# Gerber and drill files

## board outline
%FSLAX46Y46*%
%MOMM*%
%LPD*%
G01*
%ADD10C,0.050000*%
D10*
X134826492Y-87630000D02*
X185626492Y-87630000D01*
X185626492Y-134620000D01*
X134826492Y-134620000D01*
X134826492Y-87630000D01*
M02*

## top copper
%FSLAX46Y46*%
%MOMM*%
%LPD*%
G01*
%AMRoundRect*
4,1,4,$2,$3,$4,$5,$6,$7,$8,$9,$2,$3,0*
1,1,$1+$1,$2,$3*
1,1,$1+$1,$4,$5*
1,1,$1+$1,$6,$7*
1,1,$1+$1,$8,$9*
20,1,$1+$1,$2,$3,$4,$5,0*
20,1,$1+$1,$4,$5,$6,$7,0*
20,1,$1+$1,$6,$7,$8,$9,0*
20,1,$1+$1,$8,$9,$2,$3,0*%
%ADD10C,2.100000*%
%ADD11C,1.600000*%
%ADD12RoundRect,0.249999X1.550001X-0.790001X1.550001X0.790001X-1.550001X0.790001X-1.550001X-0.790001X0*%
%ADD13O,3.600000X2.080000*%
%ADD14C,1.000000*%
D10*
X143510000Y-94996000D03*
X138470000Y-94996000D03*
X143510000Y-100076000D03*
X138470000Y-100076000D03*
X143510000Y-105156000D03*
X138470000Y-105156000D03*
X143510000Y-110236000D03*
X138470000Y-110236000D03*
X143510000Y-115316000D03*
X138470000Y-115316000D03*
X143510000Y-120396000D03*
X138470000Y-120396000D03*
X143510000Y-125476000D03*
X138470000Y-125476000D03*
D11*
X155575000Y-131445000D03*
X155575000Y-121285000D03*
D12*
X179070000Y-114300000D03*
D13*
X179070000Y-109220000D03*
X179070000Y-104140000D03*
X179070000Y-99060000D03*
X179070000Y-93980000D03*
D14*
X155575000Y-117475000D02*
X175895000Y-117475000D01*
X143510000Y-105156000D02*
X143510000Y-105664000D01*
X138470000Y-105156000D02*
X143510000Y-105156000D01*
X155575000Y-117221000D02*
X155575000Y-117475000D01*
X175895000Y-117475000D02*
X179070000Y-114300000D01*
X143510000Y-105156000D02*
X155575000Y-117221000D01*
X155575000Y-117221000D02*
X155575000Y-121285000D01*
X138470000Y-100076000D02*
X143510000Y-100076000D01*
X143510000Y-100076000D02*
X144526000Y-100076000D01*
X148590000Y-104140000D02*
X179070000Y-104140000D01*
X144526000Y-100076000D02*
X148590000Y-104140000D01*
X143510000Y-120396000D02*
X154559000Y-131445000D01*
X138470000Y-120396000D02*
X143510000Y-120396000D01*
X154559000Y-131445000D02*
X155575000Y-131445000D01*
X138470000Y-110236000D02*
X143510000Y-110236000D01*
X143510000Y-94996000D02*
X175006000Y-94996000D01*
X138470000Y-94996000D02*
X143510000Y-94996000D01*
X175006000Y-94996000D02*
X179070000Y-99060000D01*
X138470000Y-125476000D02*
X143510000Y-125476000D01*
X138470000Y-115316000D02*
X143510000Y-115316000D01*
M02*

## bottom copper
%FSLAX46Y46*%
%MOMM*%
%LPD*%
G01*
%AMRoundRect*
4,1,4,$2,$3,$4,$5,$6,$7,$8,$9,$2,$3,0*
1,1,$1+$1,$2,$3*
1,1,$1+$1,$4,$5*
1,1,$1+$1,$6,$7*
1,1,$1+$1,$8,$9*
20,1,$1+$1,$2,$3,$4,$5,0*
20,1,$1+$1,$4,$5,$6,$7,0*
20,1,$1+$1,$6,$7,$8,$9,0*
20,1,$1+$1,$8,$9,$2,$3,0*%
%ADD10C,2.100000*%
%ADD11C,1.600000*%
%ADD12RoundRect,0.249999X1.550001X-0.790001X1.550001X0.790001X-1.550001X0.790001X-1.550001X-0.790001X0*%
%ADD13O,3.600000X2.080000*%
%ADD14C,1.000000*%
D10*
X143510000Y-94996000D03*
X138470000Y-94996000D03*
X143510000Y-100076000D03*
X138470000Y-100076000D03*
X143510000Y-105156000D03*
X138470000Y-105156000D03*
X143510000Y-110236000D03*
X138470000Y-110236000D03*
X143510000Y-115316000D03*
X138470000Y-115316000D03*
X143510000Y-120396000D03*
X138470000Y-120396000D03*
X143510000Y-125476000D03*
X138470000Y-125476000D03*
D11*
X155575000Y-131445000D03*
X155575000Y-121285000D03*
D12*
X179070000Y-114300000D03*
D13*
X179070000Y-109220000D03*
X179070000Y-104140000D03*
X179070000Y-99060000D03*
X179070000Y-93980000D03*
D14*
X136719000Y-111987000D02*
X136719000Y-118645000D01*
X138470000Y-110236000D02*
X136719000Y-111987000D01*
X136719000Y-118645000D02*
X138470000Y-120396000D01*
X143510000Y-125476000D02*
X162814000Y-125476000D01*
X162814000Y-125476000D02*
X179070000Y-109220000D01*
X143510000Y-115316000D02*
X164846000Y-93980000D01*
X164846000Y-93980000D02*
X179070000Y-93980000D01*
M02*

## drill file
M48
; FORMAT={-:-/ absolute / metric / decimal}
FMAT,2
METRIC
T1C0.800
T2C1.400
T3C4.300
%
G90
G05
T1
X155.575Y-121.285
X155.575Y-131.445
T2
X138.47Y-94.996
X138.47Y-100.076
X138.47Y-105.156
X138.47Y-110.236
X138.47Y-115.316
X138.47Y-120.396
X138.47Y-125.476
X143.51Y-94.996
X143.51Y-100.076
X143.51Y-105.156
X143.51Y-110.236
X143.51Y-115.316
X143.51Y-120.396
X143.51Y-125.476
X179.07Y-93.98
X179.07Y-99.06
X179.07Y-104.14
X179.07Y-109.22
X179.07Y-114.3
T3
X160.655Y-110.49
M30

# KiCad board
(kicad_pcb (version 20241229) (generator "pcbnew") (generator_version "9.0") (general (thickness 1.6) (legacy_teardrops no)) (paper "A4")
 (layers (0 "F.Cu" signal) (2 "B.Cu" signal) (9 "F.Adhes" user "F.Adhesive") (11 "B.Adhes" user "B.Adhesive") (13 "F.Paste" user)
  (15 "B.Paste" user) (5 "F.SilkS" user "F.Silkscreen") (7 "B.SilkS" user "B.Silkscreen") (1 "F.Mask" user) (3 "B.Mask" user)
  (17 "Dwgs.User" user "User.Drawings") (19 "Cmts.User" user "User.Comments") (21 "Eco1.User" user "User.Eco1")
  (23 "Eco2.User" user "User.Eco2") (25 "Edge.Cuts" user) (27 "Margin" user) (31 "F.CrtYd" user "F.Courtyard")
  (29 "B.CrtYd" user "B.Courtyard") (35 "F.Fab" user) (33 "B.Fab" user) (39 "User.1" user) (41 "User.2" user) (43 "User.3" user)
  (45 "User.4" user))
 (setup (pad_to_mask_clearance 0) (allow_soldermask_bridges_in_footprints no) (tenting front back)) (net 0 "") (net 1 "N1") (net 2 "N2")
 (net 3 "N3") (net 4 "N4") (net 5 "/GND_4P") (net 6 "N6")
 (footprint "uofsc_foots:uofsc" (layer "F.Cu") (at 177.038 124.079)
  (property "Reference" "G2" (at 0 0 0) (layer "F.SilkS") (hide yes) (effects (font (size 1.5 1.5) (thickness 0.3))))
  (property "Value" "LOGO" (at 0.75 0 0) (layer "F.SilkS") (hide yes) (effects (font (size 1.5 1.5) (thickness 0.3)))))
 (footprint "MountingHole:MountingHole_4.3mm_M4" (layer "F.Cu") (at 160.655 110.49)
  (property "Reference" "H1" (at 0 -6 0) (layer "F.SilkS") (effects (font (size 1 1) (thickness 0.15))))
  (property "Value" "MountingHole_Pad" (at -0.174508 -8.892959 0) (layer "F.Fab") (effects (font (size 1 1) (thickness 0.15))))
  (pad "" np_thru_hole circle (at 0 0) (size 4.3 4.3) (drill 4.3) (layers "*.Cu" "*.Mask")))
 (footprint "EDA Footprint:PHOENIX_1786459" (layer "F.Cu") (at 127.34 91.456 -90)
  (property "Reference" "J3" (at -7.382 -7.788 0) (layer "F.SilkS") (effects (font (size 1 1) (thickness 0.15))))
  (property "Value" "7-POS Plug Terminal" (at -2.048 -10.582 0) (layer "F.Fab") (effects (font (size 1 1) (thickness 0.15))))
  (pad "1" thru_hole circle (at 3.54 -16.17 270) (size 2.1 2.1) (drill 1.4) (layers "*.Cu" "*.Mask") (remove_unused_layers no) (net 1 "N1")
   (solder_mask_margin 0.102))
  (pad "1" thru_hole circle (at 3.54 -11.13 270) (size 2.1 2.1) (drill 1.4) (layers "*.Cu" "*.Mask") (remove_unused_layers no) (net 1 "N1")
   (solder_mask_margin 0.102))
  (pad "2" thru_hole circle (at 8.62 -16.17 270) (size 2.1 2.1) (drill 1.4) (layers "*.Cu" "*.Mask") (remove_unused_layers no) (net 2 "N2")
   (solder_mask_margin 0.102))
  (pad "2" thru_hole circle (at 8.62 -11.13 270) (size 2.1 2.1) (drill 1.4) (layers "*.Cu" "*.Mask") (remove_unused_layers no) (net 2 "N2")
   (solder_mask_margin 0.102))
  (pad "3" thru_hole circle (at 13.7 -16.17 270) (size 2.1 2.1) (drill 1.4) (layers "*.Cu" "*.Mask") (remove_unused_layers no) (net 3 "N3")
   (solder_mask_margin 0.102))
  (pad "3" thru_hole circle (at 13.7 -11.13 270) (size 2.1 2.1) (drill 1.4) (layers "*.Cu" "*.Mask") (remove_unused_layers no) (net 3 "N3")
   (solder_mask_margin 0.102))
  (pad "4" thru_hole circle (at 18.78 -16.17 270) (size 2.1 2.1) (drill 1.4) (layers "*.Cu" "*.Mask") (remove_unused_layers no) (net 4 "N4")
   (solder_mask_margin 0.102))
  (pad "4" thru_hole circle (at 18.78 -11.13 270) (size 2.1 2.1) (drill 1.4) (layers "*.Cu" "*.Mask") (remove_unused_layers no) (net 4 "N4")
   (solder_mask_margin 0.102))
  (pad "5" thru_hole circle (at 23.86 -16.17 270) (size 2.1 2.1) (drill 1.4) (layers "*.Cu" "*.Mask") (remove_unused_layers no)
   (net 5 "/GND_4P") (solder_mask_margin 0.102))
  (pad "5" thru_hole circle (at 23.86 -11.13 270) (size 2.1 2.1) (drill 1.4) (layers "*.Cu" "*.Mask") (remove_unused_layers no)
   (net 5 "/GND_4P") (solder_mask_margin 0.102))
  (pad "6" thru_hole circle (at 28.94 -16.17 270) (size 2.1 2.1) (drill 1.4) (layers "*.Cu" "*.Mask") (remove_unused_layers no) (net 4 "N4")
   (solder_mask_margin 0.102))
  (pad "6" thru_hole circle (at 28.94 -11.13 270) (size 2.1 2.1) (drill 1.4) (layers "*.Cu" "*.Mask") (remove_unused_layers no) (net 4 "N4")
   (solder_mask_margin 0.102))
  (pad "7" thru_hole circle (at 34.02 -16.17 270) (size 2.1 2.1) (drill 1.4) (layers "*.Cu" "*.Mask") (remove_unused_layers no) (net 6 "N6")
   (solder_mask_margin 0.102))
  (pad "7" thru_hole circle (at 34.02 -11.13 270) (size 2.1 2.1) (drill 1.4) (layers "*.Cu" "*.Mask") (remove_unused_layers no) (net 6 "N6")
   (solder_mask_margin 0.102)))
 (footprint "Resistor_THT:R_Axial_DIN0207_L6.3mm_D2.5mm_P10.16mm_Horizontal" (layer "F.Cu") (at 155.575 131.445 90)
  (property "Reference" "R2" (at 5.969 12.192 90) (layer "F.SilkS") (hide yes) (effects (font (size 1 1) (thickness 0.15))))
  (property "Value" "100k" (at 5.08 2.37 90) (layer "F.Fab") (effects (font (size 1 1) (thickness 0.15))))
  (pad "1" thru_hole circle (at 0 0 90) (size 1.6 1.6) (drill 0.8) (layers "*.Cu" "*.Mask") (remove_unused_layers no) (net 4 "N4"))
  (pad "2" thru_hole circle (at 10.16 0 90) (size 1.6 1.6) (drill 0.8) (layers "*.Cu" "*.Mask") (remove_unused_layers no) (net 3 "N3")))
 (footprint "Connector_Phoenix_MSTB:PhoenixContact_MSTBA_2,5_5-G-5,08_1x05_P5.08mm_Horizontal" (layer "F.Cu") (at 179.07 114.3 90)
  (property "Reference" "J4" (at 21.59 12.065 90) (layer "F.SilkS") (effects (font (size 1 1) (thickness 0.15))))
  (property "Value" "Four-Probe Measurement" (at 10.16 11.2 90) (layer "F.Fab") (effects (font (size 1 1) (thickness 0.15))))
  (pad "1" thru_hole roundrect (at 0 0 90) (size 2.08 3.6) (drill 1.4) (layers "*.Cu" "*.Mask") (remove_unused_layers no)
   (roundrect_rratio 0.120192) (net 3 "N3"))
  (pad "2" thru_hole oval (at 5.08 0 90) (size 2.08 3.6) (drill 1.4) (layers "*.Cu" "*.Mask") (remove_unused_layers no) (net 6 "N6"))
  (pad "3" thru_hole oval (at 10.16 0 90) (size 2.08 3.6) (drill 1.4) (layers "*.Cu" "*.Mask") (remove_unused_layers no) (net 2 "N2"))
  (pad "4" thru_hole oval (at 15.24 0 90) (size 2.08 3.6) (drill 1.4) (layers "*.Cu" "*.Mask") (remove_unused_layers no) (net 1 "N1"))
  (pad "5" thru_hole oval (at 20.32 0 90) (size 2.08 3.6) (drill 1.4) (layers "*.Cu" "*.Mask") (remove_unused_layers no) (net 5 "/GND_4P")))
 (gr_rect (start 134.826492 87.63) (end 185.626492 134.62) (stroke (width 0.05) (type default)) (fill no) (layer "Edge.Cuts"))
 (segment (start 155.575 117.475) (end 175.895 117.475) (width 1) (layer "F.Cu") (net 3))
 (segment (start 143.51 105.156) (end 143.51 105.664) (width 1) (layer "F.Cu") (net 3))
 (segment (start 138.47 105.156) (end 143.51 105.156) (width 1) (layer "F.Cu") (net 3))
 (segment (start 155.575 117.221) (end 155.575 117.475) (width 1) (layer "F.Cu") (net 3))
 (segment (start 175.895 117.475) (end 179.07 114.3) (width 1) (layer "F.Cu") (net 3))
 (segment (start 143.51 105.156) (end 155.575 117.221) (width 1) (layer "F.Cu") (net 3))
 (segment (start 155.575 117.221) (end 155.575 121.285) (width 1) (layer "F.Cu") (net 3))
 (segment (start 138.47 100.076) (end 143.51 100.076) (width 1) (layer "F.Cu") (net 2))
 (segment (start 143.51 100.076) (end 144.526 100.076) (width 1) (layer "F.Cu") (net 2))
 (segment (start 148.59 104.14) (end 179.07 104.14) (width 1) (layer "F.Cu") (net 2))
 (segment (start 144.526 100.076) (end 148.59 104.14) (width 1) (layer "F.Cu") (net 2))
 (segment (start 143.51 120.396) (end 154.559 131.445) (width 1) (layer "F.Cu") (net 4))
 (segment (start 138.47 120.396) (end 143.51 120.396) (width 1) (layer "F.Cu") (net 4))
 (segment (start 154.559 131.445) (end 155.575 131.445) (width 1) (layer "F.Cu") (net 4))
 (segment (start 138.47 110.236) (end 143.51 110.236) (width 1) (layer "F.Cu") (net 4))
 (segment (start 136.719 111.987) (end 136.719 118.645) (width 1) (layer "B.Cu") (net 4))
 (segment (start 138.47 110.236) (end 136.719 111.987) (width 1) (layer "B.Cu") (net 4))
 (segment (start 136.719 118.645) (end 138.47 120.396) (width 1) (layer "B.Cu") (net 4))
 (segment (start 143.51 94.996) (end 175.006 94.996) (width 1) (layer "F.Cu") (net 1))
 (segment (start 138.47 94.996) (end 143.51 94.996) (width 1) (layer "F.Cu") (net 1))
 (segment (start 175.006 94.996) (end 179.07 99.06) (width 1) (layer "F.Cu") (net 1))
 (segment (start 138.47 125.476) (end 143.51 125.476) (width 1) (layer "F.Cu") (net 6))
 (segment (start 143.51 125.476) (end 162.814 125.476) (width 1) (layer "B.Cu") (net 6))
 (segment (start 162.814 125.476) (end 179.07 109.22) (width 1) (layer "B.Cu") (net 6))
 (segment (start 138.47 115.316) (end 143.51 115.316) (width 1) (layer "F.Cu") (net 5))
 (segment (start 143.51 115.316) (end 164.846 93.98) (width 1) (layer "B.Cu") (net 5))
 (segment (start 164.846 93.98) (end 179.07 93.98) (width 1) (layer "B.Cu") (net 5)))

